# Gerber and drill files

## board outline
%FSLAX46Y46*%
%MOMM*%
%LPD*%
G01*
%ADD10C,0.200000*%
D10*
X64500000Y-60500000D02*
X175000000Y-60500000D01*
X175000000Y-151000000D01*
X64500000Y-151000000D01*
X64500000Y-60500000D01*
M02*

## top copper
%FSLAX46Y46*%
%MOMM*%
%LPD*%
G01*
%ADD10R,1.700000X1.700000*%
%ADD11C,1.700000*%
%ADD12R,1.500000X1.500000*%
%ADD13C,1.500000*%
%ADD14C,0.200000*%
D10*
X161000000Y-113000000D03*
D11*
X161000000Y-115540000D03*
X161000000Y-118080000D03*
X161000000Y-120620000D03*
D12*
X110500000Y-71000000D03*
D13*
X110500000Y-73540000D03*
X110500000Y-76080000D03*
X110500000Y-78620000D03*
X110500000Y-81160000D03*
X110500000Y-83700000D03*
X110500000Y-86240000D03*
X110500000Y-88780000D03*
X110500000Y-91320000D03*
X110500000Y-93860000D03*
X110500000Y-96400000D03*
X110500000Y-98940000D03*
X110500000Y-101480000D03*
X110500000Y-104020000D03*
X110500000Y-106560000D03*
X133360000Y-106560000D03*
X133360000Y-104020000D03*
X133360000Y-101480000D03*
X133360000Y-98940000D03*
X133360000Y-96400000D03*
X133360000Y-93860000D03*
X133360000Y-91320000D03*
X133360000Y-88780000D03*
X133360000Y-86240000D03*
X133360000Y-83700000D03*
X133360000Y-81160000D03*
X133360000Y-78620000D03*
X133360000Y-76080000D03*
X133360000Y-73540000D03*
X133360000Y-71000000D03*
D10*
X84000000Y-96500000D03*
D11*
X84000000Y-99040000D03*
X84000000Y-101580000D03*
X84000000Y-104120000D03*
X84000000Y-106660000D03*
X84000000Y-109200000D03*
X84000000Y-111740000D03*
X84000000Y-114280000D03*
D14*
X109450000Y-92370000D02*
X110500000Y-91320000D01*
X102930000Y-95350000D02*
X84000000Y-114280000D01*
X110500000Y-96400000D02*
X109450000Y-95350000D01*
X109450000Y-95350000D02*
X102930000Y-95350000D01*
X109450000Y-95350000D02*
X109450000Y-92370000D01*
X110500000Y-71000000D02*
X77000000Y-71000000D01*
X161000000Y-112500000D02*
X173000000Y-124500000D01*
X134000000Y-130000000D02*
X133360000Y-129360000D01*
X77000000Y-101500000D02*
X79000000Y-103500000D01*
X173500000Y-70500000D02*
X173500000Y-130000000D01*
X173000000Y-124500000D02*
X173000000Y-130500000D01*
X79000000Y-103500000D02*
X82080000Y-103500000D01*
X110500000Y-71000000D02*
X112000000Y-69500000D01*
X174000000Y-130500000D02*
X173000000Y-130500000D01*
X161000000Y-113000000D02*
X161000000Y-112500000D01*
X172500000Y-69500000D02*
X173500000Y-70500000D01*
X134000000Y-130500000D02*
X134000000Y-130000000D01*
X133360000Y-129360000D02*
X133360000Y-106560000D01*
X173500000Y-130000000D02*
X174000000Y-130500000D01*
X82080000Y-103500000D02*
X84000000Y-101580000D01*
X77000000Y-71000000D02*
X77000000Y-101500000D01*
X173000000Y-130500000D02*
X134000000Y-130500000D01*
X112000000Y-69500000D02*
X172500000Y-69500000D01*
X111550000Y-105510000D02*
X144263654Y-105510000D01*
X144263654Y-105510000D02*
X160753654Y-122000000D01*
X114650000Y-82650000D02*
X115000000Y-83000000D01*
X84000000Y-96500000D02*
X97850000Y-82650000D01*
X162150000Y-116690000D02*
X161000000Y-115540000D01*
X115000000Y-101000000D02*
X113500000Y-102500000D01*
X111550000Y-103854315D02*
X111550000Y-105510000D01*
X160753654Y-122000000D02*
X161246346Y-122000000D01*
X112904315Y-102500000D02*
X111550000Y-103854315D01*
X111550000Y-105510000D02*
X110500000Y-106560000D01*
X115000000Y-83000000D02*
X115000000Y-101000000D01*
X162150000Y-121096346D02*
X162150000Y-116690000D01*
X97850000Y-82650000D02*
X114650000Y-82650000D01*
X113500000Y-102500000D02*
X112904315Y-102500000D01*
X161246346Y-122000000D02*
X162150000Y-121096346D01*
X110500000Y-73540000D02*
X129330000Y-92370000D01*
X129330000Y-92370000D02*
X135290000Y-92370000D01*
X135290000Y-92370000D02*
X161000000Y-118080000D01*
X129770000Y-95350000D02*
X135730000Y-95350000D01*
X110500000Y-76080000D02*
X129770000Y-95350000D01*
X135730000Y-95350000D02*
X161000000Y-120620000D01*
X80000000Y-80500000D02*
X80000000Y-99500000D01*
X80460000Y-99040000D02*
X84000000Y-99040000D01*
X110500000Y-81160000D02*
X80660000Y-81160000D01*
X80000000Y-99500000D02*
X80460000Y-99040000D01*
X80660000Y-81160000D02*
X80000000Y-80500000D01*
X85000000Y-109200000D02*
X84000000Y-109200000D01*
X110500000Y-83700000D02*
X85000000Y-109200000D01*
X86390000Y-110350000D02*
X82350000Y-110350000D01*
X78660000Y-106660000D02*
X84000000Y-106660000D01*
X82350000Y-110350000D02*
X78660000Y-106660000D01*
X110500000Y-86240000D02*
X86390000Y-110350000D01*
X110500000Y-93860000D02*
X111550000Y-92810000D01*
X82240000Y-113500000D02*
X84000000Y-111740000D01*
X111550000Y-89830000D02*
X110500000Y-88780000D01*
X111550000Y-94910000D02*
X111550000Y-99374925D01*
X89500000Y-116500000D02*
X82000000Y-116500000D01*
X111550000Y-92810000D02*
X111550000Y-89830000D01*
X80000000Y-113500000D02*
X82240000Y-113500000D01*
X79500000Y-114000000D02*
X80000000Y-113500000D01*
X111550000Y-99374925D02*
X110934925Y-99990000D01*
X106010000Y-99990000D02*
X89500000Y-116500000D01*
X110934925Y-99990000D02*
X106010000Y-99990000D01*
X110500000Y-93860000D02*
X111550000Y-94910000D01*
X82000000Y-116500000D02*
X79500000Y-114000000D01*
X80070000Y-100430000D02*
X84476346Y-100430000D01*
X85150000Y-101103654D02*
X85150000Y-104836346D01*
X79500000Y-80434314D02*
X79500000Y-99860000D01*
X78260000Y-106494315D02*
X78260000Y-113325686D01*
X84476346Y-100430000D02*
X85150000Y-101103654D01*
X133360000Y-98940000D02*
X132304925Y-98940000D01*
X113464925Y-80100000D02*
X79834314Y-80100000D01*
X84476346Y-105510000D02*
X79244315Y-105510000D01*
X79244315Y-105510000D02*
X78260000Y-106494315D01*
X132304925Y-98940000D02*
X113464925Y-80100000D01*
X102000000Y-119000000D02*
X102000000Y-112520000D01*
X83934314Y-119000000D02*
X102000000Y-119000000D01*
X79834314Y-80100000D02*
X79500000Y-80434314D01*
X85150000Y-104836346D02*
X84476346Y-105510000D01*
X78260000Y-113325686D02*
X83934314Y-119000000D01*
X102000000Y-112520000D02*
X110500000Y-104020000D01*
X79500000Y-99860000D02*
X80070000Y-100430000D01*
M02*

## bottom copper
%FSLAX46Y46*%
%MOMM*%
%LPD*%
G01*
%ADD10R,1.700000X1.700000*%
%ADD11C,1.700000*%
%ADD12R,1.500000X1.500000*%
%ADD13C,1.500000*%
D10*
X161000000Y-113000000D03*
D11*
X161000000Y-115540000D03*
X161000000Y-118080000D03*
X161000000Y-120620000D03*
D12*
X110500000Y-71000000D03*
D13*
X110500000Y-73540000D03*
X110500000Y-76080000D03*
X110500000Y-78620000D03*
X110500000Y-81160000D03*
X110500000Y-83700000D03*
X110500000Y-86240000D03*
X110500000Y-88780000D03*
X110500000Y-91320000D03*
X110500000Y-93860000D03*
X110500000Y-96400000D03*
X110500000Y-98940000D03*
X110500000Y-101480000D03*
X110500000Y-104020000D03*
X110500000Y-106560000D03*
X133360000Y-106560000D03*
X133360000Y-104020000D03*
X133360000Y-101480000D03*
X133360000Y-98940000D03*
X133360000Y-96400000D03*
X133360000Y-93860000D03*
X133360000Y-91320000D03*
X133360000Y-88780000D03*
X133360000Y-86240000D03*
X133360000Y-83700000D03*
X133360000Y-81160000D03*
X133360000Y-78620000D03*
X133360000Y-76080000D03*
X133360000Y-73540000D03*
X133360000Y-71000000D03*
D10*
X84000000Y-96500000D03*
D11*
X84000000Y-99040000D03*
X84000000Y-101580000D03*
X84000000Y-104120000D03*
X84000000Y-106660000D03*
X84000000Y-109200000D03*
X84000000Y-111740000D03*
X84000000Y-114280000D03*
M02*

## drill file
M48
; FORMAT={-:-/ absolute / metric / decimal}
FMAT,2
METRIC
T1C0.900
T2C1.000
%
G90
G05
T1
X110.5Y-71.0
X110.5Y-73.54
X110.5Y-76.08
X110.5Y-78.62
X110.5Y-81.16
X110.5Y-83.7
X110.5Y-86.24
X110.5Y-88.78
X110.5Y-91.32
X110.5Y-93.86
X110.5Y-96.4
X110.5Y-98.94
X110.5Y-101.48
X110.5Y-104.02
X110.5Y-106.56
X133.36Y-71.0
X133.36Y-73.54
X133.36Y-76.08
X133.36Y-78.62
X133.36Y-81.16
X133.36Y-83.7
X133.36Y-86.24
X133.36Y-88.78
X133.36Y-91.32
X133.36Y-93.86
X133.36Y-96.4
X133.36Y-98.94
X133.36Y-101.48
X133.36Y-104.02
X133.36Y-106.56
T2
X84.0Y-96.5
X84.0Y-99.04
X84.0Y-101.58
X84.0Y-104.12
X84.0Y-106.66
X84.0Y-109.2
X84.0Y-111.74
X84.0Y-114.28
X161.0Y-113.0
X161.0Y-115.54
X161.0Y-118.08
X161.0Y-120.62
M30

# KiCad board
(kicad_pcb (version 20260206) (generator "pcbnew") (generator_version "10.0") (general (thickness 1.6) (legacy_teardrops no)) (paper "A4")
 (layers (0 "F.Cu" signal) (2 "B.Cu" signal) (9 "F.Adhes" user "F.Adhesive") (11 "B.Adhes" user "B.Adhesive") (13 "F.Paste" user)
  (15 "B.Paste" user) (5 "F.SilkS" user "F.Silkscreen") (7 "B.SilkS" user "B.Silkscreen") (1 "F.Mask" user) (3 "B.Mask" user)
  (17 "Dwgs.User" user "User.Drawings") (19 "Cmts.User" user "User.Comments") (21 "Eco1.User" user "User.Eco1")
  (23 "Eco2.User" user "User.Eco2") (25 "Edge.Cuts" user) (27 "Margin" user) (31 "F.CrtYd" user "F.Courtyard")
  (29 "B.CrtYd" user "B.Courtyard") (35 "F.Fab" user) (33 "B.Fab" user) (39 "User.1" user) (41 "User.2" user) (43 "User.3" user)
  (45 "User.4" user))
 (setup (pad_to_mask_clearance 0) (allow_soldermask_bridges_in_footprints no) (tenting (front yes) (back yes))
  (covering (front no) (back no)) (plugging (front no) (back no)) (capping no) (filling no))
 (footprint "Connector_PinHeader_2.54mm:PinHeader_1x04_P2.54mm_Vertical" (layer "F.Cu") (at 161 113)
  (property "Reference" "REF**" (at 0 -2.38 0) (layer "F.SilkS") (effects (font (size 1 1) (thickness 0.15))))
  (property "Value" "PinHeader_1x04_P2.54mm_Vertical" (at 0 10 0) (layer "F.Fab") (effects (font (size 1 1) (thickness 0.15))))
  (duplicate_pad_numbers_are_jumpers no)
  (pad "1" thru_hole rect (at 0 0) (size 1.7 1.7) (drill 1) (layers "*.Cu" "*.Mask") (remove_unused_layers no) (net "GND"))
  (pad "2" thru_hole circle (at 0 2.54) (size 1.7 1.7) (drill 1) (layers "*.Cu" "*.Mask") (remove_unused_layers no) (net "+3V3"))
  (pad "3" thru_hole circle (at 0 5.08) (size 1.7 1.7) (drill 1) (layers "*.Cu" "*.Mask") (remove_unused_layers no) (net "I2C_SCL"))
  (pad "4" thru_hole circle (at 0 7.62) (size 1.7 1.7) (drill 1) (layers "*.Cu" "*.Mask") (remove_unused_layers no) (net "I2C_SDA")))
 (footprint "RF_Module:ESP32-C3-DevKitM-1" (layer "F.Cu") (at 110.5 71)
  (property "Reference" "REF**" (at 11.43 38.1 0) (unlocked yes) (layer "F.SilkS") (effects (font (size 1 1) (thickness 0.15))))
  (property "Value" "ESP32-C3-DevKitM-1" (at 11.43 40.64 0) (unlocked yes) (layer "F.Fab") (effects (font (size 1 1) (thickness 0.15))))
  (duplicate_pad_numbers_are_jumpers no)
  (pad "1" thru_hole rect (at 0 0) (size 1.5 1.5) (drill 0.9) (layers "*.Cu" "*.Mask") (remove_unused_layers yes) (keep_end_layers yes)
   (zone_layer_connections) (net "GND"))
  (pad "2" thru_hole circle (at 0 2.54) (size 1.5 1.5) (drill 0.9) (layers "*.Cu" "*.Mask") (remove_unused_layers yes) (keep_end_layers yes)
   (zone_layer_connections) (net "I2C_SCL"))
  (pad "3" thru_hole circle (at 0 5.08) (size 1.5 1.5) (drill 0.9) (layers "*.Cu" "*.Mask") (remove_unused_layers yes) (keep_end_layers yes)
   (zone_layer_connections) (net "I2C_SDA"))
  (pad "4" thru_hole circle (at 0 7.62) (size 1.5 1.5) (drill 0.9) (layers "*.Cu" "*.Mask") (remove_unused_layers yes) (keep_end_layers yes)
   (zone_layer_connections) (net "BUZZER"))
  (pad "5" thru_hole circle (at 0 10.16) (size 1.5 1.5) (drill 0.9) (layers "*.Cu" "*.Mask") (remove_unused_layers yes)
   (keep_end_layers yes) (zone_layer_connections) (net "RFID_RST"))
  (pad "6" thru_hole circle (at 0 12.7) (size 1.5 1.5) (drill 0.9) (layers "*.Cu" "*.Mask") (remove_unused_layers yes) (keep_end_layers yes)
   (zone_layer_connections) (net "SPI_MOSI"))
  (pad "7" thru_hole circle (at 0 15.24) (size 1.5 1.5) (drill 0.9) (layers "*.Cu" "*.Mask") (remove_unused_layers yes)
   (keep_end_layers yes) (zone_layer_connections) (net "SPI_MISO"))
  (pad "8" thru_hole circle (at 0 17.78) (size 1.5 1.5) (drill 0.9) (layers "*.Cu" "*.Mask") (remove_unused_layers yes)
   (keep_end_layers yes) (zone_layer_connections) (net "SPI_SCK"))
  (pad "9" thru_hole circle (at 0 20.32) (size 1.5 1.5) (drill 0.9) (layers "*.Cu" "*.Mask") (remove_unused_layers yes)
   (keep_end_layers yes) (zone_layer_connections) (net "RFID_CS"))
  (pad "10" thru_hole circle (at 0 22.86) (size 1.5 1.5) (drill 0.9) (layers "*.Cu" "*.Mask") (remove_unused_layers yes)
   (keep_end_layers yes) (zone_layer_connections) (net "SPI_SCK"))
  (pad "11" thru_hole circle (at 0 25.4) (size 1.5 1.5) (drill 0.9) (layers "*.Cu" "*.Mask") (remove_unused_layers yes)
   (keep_end_layers yes) (zone_layer_connections) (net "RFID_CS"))
  (pad "12" thru_hole circle (at 0 27.94) (size 1.5 1.5) (drill 0.9) (layers "*.Cu" "*.Mask") (remove_unused_layers yes)
   (keep_end_layers yes) (zone_layer_connections))
  (pad "13" thru_hole circle (at 0 30.48) (size 1.5 1.5) (drill 0.9) (layers "*.Cu" "*.Mask") (remove_unused_layers yes)
   (keep_end_layers yes) (zone_layer_connections))
  (pad "14" thru_hole circle (at 0 33.02) (size 1.5 1.5) (drill 0.9) (layers "*.Cu" "*.Mask") (remove_unused_layers yes)
   (keep_end_layers yes) (zone_layer_connections) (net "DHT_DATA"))
  (pad "15" thru_hole circle (at 0 35.56) (size 1.5 1.5) (drill 0.9) (layers "*.Cu" "*.Mask") (remove_unused_layers yes)
   (keep_end_layers yes) (zone_layer_connections) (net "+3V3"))
  (pad "16" thru_hole circle (at 22.86 35.56) (size 1.5 1.5) (drill 0.9) (layers "*.Cu" "*.Mask") (remove_unused_layers yes)
   (keep_end_layers yes) (zone_layer_connections) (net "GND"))
  (pad "17" thru_hole circle (at 22.86 33.02) (size 1.5 1.5) (drill 0.9) (layers "*.Cu" "*.Mask") (remove_unused_layers yes)
   (keep_end_layers yes) (zone_layer_connections))
  (pad "18" thru_hole circle (at 22.86 30.48) (size 1.5 1.5) (drill 0.9) (layers "*.Cu" "*.Mask") (remove_unused_layers yes)
   (keep_end_layers yes) (zone_layer_connections))
  (pad "19" thru_hole circle (at 22.86 27.94) (size 1.5 1.5) (drill 0.9) (layers "*.Cu" "*.Mask") (remove_unused_layers yes)
   (keep_end_layers yes) (zone_layer_connections) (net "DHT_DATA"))
  (pad "20" thru_hole circle (at 22.86 25.4) (size 1.5 1.5) (drill 0.9) (layers "*.Cu" "*.Mask") (remove_unused_layers yes)
   (keep_end_layers yes) (zone_layer_connections))
  (pad "21" thru_hole circle (at 22.86 22.86) (size 1.5 1.5) (drill 0.9) (layers "*.Cu" "*.Mask") (remove_unused_layers yes)
   (keep_end_layers yes) (zone_layer_connections))
  (pad "22" thru_hole circle (at 22.86 20.32) (size 1.5 1.5) (drill 0.9) (layers "*.Cu" "*.Mask") (remove_unused_layers yes)
   (keep_end_layers yes) (zone_layer_connections) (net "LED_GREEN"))
  (pad "23" thru_hole circle (at 22.86 17.78) (size 1.5 1.5) (drill 0.9) (layers "*.Cu" "*.Mask") (remove_unused_layers yes)
   (keep_end_layers yes) (zone_layer_connections) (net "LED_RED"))
  (pad "24" thru_hole circle (at 22.86 15.24) (size 1.5 1.5) (drill 0.9) (layers "*.Cu" "*.Mask") (remove_unused_layers yes)
   (keep_end_layers yes) (zone_layer_connections))
  (pad "25" thru_hole circle (at 22.86 12.7) (size 1.5 1.5) (drill 0.9) (layers "*.Cu" "*.Mask") (remove_unused_layers yes)
   (keep_end_layers yes) (zone_layer_connections))
  (pad "26" thru_hole circle (at 22.86 10.16) (size 1.5 1.5) (drill 0.9) (layers "*.Cu" "*.Mask") (remove_unused_layers yes)
   (keep_end_layers yes) (zone_layer_connections))
  (pad "27" thru_hole circle (at 22.86 7.62) (size 1.5 1.5) (drill 0.9) (layers "*.Cu" "*.Mask") (remove_unused_layers yes)
   (keep_end_layers yes) (zone_layer_connections))
  (pad "28" thru_hole circle (at 22.86 5.08) (size 1.5 1.5) (drill 0.9) (layers "*.Cu" "*.Mask") (remove_unused_layers yes)
   (keep_end_layers yes) (zone_layer_connections))
  (pad "29" thru_hole circle (at 22.86 2.54) (size 1.5 1.5) (drill 0.9) (layers "*.Cu" "*.Mask") (remove_unused_layers yes)
   (keep_end_layers yes) (zone_layer_connections))
  (pad "30" thru_hole circle (at 22.86 0) (size 1.5 1.5) (drill 0.9) (layers "*.Cu" "*.Mask") (remove_unused_layers yes)
   (keep_end_layers yes) (zone_layer_connections)))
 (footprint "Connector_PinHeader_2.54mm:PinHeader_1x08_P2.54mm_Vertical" (layer "F.Cu") (at 84 96.5)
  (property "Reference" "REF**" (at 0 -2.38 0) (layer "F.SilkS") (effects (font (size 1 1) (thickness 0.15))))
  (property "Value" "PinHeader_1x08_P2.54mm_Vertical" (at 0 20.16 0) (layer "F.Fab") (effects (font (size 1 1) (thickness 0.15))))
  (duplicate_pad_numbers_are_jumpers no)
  (pad "1" thru_hole rect (at 0 0) (size 1.7 1.7) (drill 1) (layers "*.Cu" "*.Mask") (remove_unused_layers no) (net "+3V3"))
  (pad "2" thru_hole circle (at 0 2.54) (size 1.7 1.7) (drill 1) (layers "*.Cu" "*.Mask") (remove_unused_layers no) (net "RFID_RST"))
  (pad "3" thru_hole circle (at 0 5.08) (size 1.7 1.7) (drill 1) (layers "*.Cu" "*.Mask") (remove_unused_layers no) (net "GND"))
  (pad "4" thru_hole circle (at 0 7.62) (size 1.7 1.7) (drill 1) (layers "*.Cu" "*.Mask") (remove_unused_layers no))
  (pad "5" thru_hole circle (at 0 10.16) (size 1.7 1.7) (drill 1) (layers "*.Cu" "*.Mask") (remove_unused_layers no) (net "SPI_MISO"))
  (pad "6" thru_hole circle (at 0 12.7) (size 1.7 1.7) (drill 1) (layers "*.Cu" "*.Mask") (remove_unused_layers no) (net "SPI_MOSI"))
  (pad "7" thru_hole circle (at 0 15.24) (size 1.7 1.7) (drill 1) (layers "*.Cu" "*.Mask") (remove_unused_layers no) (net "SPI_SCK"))
  (pad "8" thru_hole circle (at 0 17.78) (size 1.7 1.7) (drill 1) (layers "*.Cu" "*.Mask") (remove_unused_layers no) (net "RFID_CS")))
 (gr_rect (start 64.5 60.5) (end 175 151) (stroke (width 0.2) (type solid)) (fill no) (layer "Edge.Cuts"))
 (segment (start 109.45 92.37) (end 110.5 91.32) (width 0.2) (layer "F.Cu") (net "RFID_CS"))
 (segment (start 102.93 95.35) (end 84 114.28) (width 0.2) (layer "F.Cu") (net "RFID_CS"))
 (segment (start 110.5 96.4) (end 109.45 95.35) (width 0.2) (layer "F.Cu") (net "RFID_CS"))
 (segment (start 109.45 95.35) (end 102.93 95.35) (width 0.2) (layer "F.Cu") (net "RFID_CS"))
 (segment (start 109.45 95.35) (end 109.45 92.37) (width 0.2) (layer "F.Cu") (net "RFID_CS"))
 (segment (start 110.5 71) (end 77 71) (width 0.2) (layer "F.Cu") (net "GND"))
 (segment (start 161 112.5) (end 173 124.5) (width 0.2) (layer "F.Cu") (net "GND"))
 (segment (start 134 130) (end 133.36 129.36) (width 0.2) (layer "F.Cu") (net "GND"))
 (segment (start 77 101.5) (end 79 103.5) (width 0.2) (layer "F.Cu") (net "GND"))
 (segment (start 173.5 70.5) (end 173.5 130) (width 0.2) (layer "F.Cu") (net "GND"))
 (segment (start 173 124.5) (end 173 130.5) (width 0.2) (layer "F.Cu") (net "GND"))
 (segment (start 79 103.5) (end 82.08 103.5) (width 0.2) (layer "F.Cu") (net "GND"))
 (segment (start 110.5 71) (end 112 69.5) (width 0.2) (layer "F.Cu") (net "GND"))
 (segment (start 174 130.5) (end 173 130.5) (width 0.2) (layer "F.Cu") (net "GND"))
 (segment (start 161 113) (end 161 112.5) (width 0.2) (layer "F.Cu") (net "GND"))
 (segment (start 172.5 69.5) (end 173.5 70.5) (width 0.2) (layer "F.Cu") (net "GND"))
 (segment (start 134 130.5) (end 134 130) (width 0.2) (layer "F.Cu") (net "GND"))
 (segment (start 133.36 129.36) (end 133.36 106.56) (width 0.2) (layer "F.Cu") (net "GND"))
 (segment (start 173.5 130) (end 174 130.5) (width 0.2) (layer "F.Cu") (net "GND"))
 (segment (start 82.08 103.5) (end 84 101.58) (width 0.2) (layer "F.Cu") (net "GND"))
 (segment (start 77 71) (end 77 101.5) (width 0.2) (layer "F.Cu") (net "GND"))
 (segment (start 173 130.5) (end 134 130.5) (width 0.2) (layer "F.Cu") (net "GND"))
 (segment (start 112 69.5) (end 172.5 69.5) (width 0.2) (layer "F.Cu") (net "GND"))
 (segment (start 111.55 105.51) (end 144.263654 105.51) (width 0.2) (layer "F.Cu") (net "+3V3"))
 (segment (start 144.263654 105.51) (end 160.753654 122) (width 0.2) (layer "F.Cu") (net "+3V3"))
 (segment (start 114.65 82.65) (end 115 83) (width 0.2) (layer "F.Cu") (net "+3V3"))
 (segment (start 84 96.5) (end 97.85 82.65) (width 0.2) (layer "F.Cu") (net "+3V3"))
 (segment (start 162.15 116.69) (end 161 115.54) (width 0.2) (layer "F.Cu") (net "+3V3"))
 (segment (start 115 101) (end 113.5 102.5) (width 0.2) (layer "F.Cu") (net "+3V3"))
 (segment (start 111.55 103.854315) (end 111.55 105.51) (width 0.2) (layer "F.Cu") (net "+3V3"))
 (segment (start 160.753654 122) (end 161.246346 122) (width 0.2) (layer "F.Cu") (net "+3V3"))
 (segment (start 112.904315 102.5) (end 111.55 103.854315) (width 0.2) (layer "F.Cu") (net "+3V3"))
 (segment (start 111.55 105.51) (end 110.5 106.56) (width 0.2) (layer "F.Cu") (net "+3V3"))
 (segment (start 115 83) (end 115 101) (width 0.2) (layer "F.Cu") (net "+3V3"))
 (segment (start 162.15 121.096346) (end 162.15 116.69) (width 0.2) (layer "F.Cu") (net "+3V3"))
 (segment (start 97.85 82.65) (end 114.65 82.65) (width 0.2) (layer "F.Cu") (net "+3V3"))
 (segment (start 113.5 102.5) (end 112.904315 102.5) (width 0.2) (layer "F.Cu") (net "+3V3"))
 (segment (start 161.246346 122) (end 162.15 121.096346) (width 0.2) (layer "F.Cu") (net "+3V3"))
 (segment (start 110.5 73.54) (end 129.33 92.37) (width 0.2) (layer "F.Cu") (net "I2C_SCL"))
 (segment (start 129.33 92.37) (end 135.29 92.37) (width 0.2) (layer "F.Cu") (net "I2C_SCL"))
 (segment (start 135.29 92.37) (end 161 118.08) (width 0.2) (layer "F.Cu") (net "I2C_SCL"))
 (segment (start 129.77 95.35) (end 135.73 95.35) (width 0.2) (layer "F.Cu") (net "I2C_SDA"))
 (segment (start 110.5 76.08) (end 129.77 95.35) (width 0.2) (layer "F.Cu") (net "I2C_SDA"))
 (segment (start 135.73 95.35) (end 161 120.62) (width 0.2) (layer "F.Cu") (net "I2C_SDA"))
 (segment (start 80 80.5) (end 80 99.5) (width 0.2) (layer "F.Cu") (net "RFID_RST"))
 (segment (start 80.46 99.04) (end 84 99.04) (width 0.2) (layer "F.Cu") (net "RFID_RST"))
 (segment (start 110.5 81.16) (end 80.66 81.16) (width 0.2) (layer "F.Cu") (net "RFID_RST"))
 (segment (start 80 99.5) (end 80.46 99.04) (width 0.2) (layer "F.Cu") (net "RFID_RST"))
 (segment (start 80.66 81.16) (end 80 80.5) (width 0.2) (layer "F.Cu") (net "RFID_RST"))
 (segment (start 85 109.2) (end 84 109.2) (width 0.2) (layer "F.Cu") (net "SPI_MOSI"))
 (segment (start 110.5 83.7) (end 85 109.2) (width 0.2) (layer "F.Cu") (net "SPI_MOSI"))
 (segment (start 86.39 110.35) (end 82.35 110.35) (width 0.2) (layer "F.Cu") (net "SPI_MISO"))
 (segment (start 78.66 106.66) (end 84 106.66) (width 0.2) (layer "F.Cu") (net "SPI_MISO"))
 (segment (start 82.35 110.35) (end 78.66 106.66) (width 0.2) (layer "F.Cu") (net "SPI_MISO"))
 (segment (start 110.5 86.24) (end 86.39 110.35) (width 0.2) (layer "F.Cu") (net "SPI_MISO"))
 (segment (start 110.5 93.86) (end 111.55 92.81) (width 0.2) (layer "F.Cu") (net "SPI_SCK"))
 (segment (start 82.24 113.5) (end 84 111.74) (width 0.2) (layer "F.Cu") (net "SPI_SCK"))
 (segment (start 111.55 89.83) (end 110.5 88.78) (width 0.2) (layer "F.Cu") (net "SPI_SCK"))
 (segment (start 111.55 94.91) (end 111.55 99.374925) (width 0.2) (layer "F.Cu") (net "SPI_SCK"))
 (segment (start 89.5 116.5) (end 82 116.5) (width 0.2) (layer "F.Cu") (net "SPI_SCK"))
 (segment (start 111.55 92.81) (end 111.55 89.83) (width 0.2) (layer "F.Cu") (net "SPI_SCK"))
 (segment (start 80 113.5) (end 82.24 113.5) (width 0.2) (layer "F.Cu") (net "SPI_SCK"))
 (segment (start 79.5 114) (end 80 113.5) (width 0.2) (layer "F.Cu") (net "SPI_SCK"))
 (segment (start 111.55 99.374925) (end 110.934925 99.99) (width 0.2) (layer "F.Cu") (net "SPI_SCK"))
 (segment (start 106.01 99.99) (end 89.5 116.5) (width 0.2) (layer "F.Cu") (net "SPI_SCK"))
 (segment (start 110.934925 99.99) (end 106.01 99.99) (width 0.2) (layer "F.Cu") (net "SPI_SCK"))
 (segment (start 110.5 93.86) (end 111.55 94.91) (width 0.2) (layer "F.Cu") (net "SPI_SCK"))
 (segment (start 82 116.5) (end 79.5 114) (width 0.2) (layer "F.Cu") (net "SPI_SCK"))
 (segment (start 80.07 100.43) (end 84.476346 100.43) (width 0.2) (layer "F.Cu") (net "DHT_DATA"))
 (segment (start 85.15 101.103654) (end 85.15 104.836346) (width 0.2) (layer "F.Cu") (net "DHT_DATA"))
 (segment (start 79.5 80.434314) (end 79.5 99.86) (width 0.2) (layer "F.Cu") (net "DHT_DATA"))
 (segment (start 78.26 106.494315) (end 78.26 113.325686) (width 0.2) (layer "F.Cu") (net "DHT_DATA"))
 (segment (start 84.476346 100.43) (end 85.15 101.103654) (width 0.2) (layer "F.Cu") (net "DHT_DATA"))
 (segment (start 133.36 98.94) (end 132.304925 98.94) (width 0.2) (layer "F.Cu") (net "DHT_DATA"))
 (segment (start 113.464925 80.1) (end 79.834314 80.1) (width 0.2) (layer "F.Cu") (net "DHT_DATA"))
 (segment (start 84.476346 105.51) (end 79.244315 105.51) (width 0.2) (layer "F.Cu") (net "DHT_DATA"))
 (segment (start 79.244315 105.51) (end 78.26 106.494315) (width 0.2) (layer "F.Cu") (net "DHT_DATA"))
 (segment (start 132.304925 98.94) (end 113.464925 80.1) (width 0.2) (layer "F.Cu") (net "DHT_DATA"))
 (segment (start 102 119) (end 102 112.52) (width 0.2) (layer "F.Cu") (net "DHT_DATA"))
 (segment (start 83.934314 119) (end 102 119) (width 0.2) (layer "F.Cu") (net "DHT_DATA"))
 (segment (start 79.834314 80.1) (end 79.5 80.434314) (width 0.2) (layer "F.Cu") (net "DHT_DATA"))
 (segment (start 85.15 104.836346) (end 84.476346 105.51) (width 0.2) (layer "F.Cu") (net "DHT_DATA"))
 (segment (start 78.26 113.325686) (end 83.934314 119) (width 0.2) (layer "F.Cu") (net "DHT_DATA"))
 (segment (start 102 112.52) (end 110.5 104.02) (width 0.2) (layer "F.Cu") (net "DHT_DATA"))
 (segment (start 79.5 99.86) (end 80.07 100.43) (width 0.2) (layer "F.Cu") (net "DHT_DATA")))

